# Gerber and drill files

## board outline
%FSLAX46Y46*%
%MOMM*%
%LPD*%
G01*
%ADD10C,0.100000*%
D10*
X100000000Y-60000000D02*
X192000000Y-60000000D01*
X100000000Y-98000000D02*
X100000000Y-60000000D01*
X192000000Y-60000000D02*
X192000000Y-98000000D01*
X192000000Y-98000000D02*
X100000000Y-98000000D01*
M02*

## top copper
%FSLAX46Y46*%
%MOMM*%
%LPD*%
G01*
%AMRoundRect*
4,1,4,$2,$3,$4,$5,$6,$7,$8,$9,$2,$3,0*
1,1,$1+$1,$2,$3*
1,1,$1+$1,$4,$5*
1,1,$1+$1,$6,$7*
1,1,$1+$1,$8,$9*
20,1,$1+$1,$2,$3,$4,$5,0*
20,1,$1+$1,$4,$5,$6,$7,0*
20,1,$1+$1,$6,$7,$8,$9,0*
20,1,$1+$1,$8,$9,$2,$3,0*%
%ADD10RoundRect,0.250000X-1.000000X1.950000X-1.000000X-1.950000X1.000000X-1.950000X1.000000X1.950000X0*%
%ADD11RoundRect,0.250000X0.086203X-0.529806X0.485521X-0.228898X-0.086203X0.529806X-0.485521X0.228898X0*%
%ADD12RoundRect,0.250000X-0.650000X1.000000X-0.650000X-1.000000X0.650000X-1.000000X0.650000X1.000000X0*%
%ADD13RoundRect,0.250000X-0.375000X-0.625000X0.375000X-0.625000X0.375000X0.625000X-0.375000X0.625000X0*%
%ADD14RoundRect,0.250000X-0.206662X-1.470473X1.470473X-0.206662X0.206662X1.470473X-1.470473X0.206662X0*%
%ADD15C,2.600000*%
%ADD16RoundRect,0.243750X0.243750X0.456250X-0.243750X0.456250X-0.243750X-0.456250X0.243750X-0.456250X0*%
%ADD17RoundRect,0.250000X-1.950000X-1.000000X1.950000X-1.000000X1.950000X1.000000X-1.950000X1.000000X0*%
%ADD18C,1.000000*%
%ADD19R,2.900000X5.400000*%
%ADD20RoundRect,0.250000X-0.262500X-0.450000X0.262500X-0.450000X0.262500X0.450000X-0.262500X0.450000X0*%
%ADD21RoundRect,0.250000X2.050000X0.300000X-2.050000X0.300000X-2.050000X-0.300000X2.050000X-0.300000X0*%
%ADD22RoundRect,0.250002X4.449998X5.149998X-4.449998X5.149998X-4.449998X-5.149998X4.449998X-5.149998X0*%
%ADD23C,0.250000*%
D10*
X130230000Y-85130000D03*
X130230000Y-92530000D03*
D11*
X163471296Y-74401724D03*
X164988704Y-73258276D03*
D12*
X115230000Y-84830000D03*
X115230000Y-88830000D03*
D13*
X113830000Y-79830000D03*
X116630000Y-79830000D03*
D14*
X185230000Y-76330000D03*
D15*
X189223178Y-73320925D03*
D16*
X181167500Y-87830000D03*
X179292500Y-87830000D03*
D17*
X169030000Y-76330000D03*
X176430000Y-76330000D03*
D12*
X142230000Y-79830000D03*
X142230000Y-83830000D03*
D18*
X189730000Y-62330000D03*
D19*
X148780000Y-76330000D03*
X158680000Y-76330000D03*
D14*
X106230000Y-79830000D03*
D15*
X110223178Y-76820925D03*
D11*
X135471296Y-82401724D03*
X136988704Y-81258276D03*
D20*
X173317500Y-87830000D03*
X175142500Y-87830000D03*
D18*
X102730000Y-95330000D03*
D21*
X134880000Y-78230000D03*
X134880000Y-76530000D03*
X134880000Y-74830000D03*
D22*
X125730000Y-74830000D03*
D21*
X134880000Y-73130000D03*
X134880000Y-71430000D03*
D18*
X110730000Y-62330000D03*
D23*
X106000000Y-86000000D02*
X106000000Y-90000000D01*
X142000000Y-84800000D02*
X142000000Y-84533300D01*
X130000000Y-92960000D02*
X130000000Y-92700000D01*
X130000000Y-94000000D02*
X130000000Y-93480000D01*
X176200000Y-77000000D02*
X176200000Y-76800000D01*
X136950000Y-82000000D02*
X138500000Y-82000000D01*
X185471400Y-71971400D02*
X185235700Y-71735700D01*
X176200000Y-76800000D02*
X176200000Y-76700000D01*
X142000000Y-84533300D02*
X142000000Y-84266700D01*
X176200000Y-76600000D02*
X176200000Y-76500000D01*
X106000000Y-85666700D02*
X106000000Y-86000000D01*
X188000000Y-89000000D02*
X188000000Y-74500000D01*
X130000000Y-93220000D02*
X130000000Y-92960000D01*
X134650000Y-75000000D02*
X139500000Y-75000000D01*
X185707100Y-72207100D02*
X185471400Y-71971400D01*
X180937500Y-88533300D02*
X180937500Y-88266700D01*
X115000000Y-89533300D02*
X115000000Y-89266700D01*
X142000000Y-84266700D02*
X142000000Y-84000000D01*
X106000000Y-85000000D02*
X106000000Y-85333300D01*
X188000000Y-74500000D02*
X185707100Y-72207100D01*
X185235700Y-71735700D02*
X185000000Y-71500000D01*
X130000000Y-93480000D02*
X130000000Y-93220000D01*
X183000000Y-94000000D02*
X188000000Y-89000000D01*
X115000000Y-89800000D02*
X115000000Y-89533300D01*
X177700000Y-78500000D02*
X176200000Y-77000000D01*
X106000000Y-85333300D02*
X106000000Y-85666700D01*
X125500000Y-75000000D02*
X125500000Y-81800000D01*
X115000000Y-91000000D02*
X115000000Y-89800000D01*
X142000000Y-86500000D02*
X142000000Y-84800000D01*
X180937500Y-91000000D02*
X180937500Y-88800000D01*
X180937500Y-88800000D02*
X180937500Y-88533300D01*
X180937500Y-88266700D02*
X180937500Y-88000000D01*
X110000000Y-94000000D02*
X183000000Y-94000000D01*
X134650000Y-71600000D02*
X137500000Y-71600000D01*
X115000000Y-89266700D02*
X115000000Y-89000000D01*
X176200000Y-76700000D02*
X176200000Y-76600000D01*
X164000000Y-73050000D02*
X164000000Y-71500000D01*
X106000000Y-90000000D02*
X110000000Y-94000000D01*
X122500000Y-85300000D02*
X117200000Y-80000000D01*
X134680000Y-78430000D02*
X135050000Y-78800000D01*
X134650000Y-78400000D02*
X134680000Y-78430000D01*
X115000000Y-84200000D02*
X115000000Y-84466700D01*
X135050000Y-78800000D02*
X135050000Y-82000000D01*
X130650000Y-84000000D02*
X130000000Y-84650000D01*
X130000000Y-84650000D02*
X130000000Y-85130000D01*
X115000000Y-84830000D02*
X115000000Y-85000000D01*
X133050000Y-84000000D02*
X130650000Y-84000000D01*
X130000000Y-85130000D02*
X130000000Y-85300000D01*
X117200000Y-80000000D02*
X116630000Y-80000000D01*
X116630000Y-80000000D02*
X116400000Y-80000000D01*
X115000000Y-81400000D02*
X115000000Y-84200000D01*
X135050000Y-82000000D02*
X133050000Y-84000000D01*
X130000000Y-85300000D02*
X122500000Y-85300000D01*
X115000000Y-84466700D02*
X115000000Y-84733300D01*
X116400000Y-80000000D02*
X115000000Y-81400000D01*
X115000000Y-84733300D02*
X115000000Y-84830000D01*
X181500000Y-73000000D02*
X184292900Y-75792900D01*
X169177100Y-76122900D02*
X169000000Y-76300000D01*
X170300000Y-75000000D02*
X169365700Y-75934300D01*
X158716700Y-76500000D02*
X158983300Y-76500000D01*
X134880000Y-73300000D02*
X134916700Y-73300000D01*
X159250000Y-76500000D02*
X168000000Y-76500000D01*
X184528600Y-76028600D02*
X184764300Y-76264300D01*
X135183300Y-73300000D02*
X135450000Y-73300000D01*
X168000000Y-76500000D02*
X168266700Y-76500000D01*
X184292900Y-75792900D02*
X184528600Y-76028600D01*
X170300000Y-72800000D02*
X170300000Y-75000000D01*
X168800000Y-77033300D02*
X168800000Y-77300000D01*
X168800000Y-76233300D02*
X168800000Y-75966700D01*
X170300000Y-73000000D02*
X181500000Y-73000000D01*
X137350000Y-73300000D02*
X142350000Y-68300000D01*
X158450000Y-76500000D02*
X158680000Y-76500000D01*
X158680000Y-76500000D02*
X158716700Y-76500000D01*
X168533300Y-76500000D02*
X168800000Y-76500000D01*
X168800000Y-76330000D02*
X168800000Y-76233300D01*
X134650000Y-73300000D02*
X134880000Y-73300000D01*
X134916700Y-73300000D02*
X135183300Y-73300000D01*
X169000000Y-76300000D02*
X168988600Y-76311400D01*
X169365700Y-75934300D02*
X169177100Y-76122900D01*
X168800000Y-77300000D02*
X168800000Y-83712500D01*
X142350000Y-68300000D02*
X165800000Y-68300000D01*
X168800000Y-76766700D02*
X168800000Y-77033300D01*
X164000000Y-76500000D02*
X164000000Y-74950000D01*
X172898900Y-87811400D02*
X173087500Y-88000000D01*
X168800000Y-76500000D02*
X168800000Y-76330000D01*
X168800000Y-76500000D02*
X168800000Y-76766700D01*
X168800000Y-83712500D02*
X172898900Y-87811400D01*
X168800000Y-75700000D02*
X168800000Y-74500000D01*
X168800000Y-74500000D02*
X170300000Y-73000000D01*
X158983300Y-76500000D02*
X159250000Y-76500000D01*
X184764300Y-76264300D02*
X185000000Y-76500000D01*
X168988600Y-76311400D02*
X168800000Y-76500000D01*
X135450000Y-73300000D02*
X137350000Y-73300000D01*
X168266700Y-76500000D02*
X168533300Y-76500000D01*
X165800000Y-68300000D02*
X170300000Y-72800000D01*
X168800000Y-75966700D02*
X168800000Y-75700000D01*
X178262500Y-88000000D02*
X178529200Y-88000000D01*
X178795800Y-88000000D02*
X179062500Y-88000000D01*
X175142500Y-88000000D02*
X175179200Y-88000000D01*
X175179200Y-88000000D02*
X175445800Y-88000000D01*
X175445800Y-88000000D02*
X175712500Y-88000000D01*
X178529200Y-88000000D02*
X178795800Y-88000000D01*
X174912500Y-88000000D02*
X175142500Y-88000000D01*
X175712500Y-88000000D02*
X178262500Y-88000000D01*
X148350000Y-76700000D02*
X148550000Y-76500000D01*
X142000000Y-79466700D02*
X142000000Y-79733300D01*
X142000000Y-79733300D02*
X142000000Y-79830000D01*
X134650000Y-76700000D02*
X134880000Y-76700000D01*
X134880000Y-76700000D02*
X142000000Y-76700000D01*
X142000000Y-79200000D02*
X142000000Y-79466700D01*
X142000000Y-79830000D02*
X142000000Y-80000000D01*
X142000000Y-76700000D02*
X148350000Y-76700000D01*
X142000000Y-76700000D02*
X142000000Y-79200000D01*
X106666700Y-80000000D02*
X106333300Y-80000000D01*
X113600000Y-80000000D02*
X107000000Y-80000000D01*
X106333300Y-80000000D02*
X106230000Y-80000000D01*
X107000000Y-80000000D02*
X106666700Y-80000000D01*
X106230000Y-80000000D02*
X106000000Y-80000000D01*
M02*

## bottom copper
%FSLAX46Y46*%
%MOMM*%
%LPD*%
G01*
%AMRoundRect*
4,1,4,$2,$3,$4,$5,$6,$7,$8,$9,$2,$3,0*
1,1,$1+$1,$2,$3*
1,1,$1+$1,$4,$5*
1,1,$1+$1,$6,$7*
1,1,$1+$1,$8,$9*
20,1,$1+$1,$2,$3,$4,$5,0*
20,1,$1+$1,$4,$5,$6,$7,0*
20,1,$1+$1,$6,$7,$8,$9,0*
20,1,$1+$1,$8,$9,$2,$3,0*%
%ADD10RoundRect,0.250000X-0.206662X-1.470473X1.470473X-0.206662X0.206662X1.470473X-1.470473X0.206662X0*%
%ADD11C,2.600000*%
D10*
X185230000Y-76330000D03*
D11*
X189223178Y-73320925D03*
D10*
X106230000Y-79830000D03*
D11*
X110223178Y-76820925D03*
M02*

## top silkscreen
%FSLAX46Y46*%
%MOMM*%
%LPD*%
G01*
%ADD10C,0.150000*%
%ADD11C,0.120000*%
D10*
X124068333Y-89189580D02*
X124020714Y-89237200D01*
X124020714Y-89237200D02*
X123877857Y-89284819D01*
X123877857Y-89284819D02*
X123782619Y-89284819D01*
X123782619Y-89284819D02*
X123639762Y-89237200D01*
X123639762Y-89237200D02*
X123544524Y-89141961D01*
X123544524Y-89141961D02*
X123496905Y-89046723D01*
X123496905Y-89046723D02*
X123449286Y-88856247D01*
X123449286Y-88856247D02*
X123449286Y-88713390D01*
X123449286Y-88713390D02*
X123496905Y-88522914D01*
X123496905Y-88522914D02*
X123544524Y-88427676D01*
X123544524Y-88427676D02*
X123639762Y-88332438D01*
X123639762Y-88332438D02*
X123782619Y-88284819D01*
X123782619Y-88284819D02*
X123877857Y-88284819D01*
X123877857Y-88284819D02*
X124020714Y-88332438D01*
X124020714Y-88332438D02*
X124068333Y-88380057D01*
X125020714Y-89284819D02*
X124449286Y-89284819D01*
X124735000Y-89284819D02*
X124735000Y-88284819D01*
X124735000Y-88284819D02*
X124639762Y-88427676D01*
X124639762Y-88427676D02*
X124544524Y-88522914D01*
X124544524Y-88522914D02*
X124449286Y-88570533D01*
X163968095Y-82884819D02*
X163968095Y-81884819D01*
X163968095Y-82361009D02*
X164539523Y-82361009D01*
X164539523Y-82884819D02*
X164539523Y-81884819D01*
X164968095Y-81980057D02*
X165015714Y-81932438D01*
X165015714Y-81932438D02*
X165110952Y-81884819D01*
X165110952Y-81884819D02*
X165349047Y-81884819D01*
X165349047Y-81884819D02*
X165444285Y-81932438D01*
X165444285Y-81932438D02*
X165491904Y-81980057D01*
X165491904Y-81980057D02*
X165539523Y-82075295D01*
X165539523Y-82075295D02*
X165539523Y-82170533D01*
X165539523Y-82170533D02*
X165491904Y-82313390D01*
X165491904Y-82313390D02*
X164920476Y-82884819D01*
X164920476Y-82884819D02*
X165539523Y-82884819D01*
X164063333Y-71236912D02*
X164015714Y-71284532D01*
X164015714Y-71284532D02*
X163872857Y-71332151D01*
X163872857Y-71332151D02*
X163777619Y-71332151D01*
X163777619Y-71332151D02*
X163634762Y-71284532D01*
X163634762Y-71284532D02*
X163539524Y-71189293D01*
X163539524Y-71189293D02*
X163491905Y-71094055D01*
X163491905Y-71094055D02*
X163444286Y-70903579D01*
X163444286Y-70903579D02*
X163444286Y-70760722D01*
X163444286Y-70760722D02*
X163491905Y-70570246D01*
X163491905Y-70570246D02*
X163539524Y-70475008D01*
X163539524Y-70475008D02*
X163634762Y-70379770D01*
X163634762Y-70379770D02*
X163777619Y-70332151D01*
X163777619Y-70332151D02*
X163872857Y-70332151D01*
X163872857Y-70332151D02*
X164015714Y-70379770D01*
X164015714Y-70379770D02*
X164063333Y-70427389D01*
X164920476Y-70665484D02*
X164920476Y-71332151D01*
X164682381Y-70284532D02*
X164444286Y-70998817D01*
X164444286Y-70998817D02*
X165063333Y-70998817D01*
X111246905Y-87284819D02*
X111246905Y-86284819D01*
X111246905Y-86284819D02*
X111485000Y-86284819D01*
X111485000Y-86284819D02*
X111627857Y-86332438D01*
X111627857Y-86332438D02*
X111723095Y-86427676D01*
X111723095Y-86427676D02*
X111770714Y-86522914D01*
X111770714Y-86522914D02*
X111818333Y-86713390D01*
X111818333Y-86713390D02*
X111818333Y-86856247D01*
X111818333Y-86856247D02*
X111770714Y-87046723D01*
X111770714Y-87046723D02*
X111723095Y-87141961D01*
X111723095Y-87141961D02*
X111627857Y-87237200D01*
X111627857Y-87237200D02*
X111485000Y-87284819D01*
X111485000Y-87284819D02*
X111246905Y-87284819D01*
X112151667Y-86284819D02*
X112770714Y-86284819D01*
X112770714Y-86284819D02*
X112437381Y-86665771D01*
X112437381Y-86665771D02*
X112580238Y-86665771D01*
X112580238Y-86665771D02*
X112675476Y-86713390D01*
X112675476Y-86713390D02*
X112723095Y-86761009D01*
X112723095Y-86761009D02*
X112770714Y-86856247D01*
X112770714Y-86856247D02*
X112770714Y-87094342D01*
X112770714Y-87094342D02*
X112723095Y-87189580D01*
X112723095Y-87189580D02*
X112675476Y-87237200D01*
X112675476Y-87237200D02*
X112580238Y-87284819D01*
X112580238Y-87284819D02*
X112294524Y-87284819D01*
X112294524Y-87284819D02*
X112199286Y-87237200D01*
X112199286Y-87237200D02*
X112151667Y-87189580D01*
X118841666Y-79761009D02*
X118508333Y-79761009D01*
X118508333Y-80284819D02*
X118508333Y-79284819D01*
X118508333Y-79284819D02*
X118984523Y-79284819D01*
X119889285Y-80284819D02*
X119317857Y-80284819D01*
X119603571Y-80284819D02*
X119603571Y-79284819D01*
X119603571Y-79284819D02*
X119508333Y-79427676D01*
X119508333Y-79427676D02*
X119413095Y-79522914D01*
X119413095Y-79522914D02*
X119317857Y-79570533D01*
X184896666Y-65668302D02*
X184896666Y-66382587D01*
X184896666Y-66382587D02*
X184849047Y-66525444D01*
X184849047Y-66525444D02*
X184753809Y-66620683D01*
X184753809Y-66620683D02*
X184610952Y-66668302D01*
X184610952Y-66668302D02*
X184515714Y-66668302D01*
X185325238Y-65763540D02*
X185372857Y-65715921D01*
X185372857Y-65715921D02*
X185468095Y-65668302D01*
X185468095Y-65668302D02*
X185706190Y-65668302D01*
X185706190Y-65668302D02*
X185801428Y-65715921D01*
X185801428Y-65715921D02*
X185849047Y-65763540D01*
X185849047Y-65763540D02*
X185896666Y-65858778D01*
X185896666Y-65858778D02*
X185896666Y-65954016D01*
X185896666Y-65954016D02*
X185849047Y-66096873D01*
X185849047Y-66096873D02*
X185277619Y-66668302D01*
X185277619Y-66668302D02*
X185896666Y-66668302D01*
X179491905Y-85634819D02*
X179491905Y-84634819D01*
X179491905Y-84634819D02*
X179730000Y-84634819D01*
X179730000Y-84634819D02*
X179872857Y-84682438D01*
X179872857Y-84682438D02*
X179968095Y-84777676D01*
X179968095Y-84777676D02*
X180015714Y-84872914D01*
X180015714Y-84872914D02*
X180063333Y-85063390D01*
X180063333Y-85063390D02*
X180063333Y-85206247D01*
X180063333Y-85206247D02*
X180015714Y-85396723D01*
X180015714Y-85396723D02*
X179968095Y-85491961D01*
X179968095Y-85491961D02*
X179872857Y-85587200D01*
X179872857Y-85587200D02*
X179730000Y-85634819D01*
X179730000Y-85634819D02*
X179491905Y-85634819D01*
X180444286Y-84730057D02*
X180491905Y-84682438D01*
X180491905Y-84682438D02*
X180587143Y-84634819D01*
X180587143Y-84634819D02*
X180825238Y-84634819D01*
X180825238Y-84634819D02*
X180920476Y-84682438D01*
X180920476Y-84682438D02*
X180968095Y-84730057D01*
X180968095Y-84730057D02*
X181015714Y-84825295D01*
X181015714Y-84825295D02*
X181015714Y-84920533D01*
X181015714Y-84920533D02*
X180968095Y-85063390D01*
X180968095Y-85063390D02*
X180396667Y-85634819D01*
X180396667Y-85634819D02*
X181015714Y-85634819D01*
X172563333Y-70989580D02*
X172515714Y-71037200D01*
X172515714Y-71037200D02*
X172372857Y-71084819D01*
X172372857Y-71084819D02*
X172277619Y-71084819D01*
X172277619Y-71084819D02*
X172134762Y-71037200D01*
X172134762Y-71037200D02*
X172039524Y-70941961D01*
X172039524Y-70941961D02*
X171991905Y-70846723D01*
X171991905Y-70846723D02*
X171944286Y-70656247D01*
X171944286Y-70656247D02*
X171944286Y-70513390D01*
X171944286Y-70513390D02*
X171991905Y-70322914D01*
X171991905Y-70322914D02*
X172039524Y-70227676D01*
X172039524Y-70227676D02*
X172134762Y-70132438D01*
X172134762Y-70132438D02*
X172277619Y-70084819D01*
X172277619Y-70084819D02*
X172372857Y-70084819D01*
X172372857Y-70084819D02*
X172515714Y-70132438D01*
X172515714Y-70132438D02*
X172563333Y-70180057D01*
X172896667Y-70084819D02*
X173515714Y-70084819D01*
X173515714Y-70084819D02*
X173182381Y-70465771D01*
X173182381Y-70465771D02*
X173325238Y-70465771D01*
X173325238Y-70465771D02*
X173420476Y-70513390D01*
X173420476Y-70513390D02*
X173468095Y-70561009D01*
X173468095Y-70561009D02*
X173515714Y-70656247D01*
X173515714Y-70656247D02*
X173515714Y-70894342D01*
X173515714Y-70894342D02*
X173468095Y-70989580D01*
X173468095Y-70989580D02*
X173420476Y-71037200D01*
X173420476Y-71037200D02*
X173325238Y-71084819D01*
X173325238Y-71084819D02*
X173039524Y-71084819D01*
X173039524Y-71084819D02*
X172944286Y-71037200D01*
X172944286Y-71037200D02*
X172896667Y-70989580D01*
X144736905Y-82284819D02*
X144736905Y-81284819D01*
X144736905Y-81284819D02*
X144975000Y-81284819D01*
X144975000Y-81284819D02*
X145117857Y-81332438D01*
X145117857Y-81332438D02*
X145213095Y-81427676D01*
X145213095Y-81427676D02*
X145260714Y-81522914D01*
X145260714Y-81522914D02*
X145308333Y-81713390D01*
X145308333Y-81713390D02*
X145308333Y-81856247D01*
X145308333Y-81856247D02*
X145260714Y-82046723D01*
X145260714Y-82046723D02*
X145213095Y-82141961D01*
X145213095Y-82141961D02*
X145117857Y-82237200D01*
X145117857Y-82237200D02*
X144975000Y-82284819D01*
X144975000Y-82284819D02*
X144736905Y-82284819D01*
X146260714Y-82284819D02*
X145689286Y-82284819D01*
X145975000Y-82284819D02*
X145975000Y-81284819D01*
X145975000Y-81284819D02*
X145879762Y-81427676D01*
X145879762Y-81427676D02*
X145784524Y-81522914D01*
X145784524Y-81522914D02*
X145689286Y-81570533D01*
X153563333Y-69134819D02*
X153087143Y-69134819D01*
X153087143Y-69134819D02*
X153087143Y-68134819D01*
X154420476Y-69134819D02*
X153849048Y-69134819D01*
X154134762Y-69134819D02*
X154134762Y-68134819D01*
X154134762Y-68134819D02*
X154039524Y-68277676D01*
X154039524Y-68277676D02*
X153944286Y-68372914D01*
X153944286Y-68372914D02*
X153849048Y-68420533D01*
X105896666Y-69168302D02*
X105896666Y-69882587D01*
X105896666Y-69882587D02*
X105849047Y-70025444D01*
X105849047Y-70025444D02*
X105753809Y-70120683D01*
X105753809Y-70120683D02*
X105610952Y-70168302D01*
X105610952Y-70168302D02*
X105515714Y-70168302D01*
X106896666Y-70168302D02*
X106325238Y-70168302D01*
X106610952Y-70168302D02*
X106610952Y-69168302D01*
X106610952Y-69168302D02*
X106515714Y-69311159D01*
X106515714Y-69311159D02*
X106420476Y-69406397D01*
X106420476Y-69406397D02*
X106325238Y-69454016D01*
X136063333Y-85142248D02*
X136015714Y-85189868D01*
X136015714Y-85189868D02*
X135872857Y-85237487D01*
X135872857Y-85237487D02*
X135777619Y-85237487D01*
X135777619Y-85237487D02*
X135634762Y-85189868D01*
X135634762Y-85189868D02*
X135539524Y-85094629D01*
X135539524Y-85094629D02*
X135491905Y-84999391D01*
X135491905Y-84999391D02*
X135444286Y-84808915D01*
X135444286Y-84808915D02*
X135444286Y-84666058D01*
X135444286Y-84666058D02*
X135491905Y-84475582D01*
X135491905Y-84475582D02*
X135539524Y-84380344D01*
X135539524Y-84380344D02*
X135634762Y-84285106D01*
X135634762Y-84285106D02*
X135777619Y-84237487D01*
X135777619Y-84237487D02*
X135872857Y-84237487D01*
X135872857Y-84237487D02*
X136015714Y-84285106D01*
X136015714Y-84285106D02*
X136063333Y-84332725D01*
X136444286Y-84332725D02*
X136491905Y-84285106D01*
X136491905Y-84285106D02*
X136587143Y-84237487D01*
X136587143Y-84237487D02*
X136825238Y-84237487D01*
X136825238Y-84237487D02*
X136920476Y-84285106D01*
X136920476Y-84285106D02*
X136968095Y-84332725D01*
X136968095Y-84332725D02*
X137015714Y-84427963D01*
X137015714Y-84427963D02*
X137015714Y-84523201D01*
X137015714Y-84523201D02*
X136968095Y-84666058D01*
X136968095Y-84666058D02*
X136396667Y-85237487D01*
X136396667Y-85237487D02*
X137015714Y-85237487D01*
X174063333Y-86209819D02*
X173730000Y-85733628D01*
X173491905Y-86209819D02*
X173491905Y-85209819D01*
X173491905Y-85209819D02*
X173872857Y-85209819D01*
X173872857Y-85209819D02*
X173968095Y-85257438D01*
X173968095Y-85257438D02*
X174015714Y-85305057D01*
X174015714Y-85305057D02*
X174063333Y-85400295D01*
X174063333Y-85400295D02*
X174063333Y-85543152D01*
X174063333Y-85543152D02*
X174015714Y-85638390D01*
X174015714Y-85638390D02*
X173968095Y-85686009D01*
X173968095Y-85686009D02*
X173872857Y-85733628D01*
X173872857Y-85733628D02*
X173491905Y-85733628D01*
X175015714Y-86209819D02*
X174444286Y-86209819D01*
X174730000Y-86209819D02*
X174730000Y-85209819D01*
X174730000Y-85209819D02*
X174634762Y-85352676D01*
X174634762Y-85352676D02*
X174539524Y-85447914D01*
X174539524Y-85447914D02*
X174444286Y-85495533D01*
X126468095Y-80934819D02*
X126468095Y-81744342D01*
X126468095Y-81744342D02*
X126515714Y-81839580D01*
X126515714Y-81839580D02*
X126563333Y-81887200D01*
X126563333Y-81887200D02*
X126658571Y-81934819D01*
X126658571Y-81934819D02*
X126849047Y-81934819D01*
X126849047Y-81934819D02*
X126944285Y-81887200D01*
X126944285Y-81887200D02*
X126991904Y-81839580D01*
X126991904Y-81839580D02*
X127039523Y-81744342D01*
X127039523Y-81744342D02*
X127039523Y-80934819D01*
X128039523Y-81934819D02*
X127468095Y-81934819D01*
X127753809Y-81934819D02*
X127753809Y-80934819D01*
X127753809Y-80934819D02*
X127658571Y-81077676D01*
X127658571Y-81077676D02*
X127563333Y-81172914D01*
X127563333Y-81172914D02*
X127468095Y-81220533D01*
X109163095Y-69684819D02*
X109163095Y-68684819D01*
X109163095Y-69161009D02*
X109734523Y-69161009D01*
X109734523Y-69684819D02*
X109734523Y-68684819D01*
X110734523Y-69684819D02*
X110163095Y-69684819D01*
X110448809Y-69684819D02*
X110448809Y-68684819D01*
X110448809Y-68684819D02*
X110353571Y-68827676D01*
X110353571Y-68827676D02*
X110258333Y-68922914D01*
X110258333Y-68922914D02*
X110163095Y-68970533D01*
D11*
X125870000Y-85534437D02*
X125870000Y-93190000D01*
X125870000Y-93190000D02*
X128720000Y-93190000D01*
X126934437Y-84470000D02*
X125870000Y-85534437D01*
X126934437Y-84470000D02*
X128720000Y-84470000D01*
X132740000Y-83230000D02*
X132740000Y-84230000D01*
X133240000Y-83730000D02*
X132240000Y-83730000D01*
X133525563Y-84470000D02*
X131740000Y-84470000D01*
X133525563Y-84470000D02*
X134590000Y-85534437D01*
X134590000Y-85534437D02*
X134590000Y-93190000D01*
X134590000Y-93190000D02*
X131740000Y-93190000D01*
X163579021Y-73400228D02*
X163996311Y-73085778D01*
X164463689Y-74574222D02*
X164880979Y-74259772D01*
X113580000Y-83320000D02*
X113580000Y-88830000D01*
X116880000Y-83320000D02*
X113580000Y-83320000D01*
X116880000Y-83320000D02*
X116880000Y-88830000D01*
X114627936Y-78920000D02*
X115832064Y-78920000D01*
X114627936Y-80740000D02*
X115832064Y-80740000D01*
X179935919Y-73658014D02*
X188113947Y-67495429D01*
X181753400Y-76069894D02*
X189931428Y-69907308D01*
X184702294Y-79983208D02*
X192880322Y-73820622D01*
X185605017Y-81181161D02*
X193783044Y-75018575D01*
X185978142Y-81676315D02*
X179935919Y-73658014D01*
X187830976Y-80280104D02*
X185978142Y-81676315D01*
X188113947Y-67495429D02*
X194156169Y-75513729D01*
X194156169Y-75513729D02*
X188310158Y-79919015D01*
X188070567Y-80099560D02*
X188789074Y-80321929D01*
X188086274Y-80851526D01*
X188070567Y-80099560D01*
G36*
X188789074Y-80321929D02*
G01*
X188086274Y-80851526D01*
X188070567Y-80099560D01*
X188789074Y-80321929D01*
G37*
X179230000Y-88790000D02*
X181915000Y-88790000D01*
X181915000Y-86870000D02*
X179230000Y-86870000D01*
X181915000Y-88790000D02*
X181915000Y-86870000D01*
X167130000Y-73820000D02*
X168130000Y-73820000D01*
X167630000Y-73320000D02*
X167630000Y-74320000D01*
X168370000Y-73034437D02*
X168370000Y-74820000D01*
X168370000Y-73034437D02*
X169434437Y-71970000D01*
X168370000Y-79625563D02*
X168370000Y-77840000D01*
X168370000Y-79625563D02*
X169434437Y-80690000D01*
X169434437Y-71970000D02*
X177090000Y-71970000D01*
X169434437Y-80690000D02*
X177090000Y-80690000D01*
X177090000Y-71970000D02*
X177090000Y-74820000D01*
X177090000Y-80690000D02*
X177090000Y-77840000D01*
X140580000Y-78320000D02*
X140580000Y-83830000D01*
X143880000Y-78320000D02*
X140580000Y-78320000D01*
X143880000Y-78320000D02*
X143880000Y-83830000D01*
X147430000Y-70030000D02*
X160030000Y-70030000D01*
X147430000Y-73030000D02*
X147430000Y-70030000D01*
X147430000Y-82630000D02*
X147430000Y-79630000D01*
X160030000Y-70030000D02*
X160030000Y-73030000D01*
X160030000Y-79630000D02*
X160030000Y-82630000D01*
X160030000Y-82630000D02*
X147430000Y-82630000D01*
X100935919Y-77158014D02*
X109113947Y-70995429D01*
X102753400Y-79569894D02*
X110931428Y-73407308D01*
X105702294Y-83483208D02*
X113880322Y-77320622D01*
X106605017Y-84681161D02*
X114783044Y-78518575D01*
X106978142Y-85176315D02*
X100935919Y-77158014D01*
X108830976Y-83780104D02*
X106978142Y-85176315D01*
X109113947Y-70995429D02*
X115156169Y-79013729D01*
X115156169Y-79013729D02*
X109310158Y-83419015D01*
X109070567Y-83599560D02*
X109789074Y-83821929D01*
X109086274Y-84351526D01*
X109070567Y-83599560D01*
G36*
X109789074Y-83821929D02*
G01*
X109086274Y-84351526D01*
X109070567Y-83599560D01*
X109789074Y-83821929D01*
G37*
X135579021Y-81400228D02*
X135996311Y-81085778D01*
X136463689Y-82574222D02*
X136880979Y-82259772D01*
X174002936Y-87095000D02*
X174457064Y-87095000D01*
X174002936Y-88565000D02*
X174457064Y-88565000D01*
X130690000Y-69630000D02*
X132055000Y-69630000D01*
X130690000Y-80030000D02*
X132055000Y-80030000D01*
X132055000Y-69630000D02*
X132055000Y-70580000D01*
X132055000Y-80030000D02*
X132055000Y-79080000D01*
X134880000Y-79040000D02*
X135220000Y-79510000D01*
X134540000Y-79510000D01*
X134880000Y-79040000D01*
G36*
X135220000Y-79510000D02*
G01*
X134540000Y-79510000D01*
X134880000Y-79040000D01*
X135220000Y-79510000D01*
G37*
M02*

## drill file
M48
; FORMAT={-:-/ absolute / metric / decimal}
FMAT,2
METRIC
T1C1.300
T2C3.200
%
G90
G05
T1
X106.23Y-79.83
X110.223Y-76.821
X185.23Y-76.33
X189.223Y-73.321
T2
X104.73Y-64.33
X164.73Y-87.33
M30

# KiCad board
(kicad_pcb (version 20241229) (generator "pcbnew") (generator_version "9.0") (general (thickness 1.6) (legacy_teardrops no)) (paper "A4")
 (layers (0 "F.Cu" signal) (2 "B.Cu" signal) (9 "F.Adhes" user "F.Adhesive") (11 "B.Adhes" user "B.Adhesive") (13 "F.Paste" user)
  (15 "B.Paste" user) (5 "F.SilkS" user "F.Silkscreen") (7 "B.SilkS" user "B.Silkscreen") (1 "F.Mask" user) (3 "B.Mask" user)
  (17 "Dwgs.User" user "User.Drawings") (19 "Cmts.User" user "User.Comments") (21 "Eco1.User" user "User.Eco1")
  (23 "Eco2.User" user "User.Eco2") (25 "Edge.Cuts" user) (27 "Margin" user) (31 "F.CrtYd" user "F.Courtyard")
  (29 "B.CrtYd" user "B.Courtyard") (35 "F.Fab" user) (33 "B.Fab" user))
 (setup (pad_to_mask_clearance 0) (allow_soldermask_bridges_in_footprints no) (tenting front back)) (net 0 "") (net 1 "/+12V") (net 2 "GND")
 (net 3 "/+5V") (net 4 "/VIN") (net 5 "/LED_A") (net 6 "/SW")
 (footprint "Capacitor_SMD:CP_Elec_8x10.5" (layer "F.Cu") (at 130.23 88.83 -90)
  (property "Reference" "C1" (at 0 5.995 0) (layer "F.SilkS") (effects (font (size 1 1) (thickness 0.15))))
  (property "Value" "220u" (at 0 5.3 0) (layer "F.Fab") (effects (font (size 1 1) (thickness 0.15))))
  (fp_line (start -3.295563 4.36) (end 4.36 4.36) (stroke (width 0.12) (type solid)) (layer "F.SilkS"))
  (fp_line (start 4.36 4.36) (end 4.36 1.51) (stroke (width 0.12) (type solid)) (layer "F.SilkS"))
  (fp_line (start -4.36 3.295563) (end -3.295563 4.36) (stroke (width 0.12) (type solid)) (layer "F.SilkS"))
  (fp_line (start -4.36 3.295563) (end -4.36 1.51) (stroke (width 0.12) (type solid)) (layer "F.SilkS"))
  (fp_line (start -5.6 -2.51) (end -4.6 -2.51) (stroke (width 0.12) (type solid)) (layer "F.SilkS"))
  (fp_line (start -5.1 -3.01) (end -5.1 -2.01) (stroke (width 0.12) (type solid)) (layer "F.SilkS"))
  (fp_line (start -4.36 -3.295563) (end -4.36 -1.51) (stroke (width 0.12) (type solid)) (layer "F.SilkS"))
  (fp_line (start -4.36 -3.295563) (end -3.295563 -4.36) (stroke (width 0.12) (type solid)) (layer "F.SilkS"))
  (fp_line (start -3.295563 -4.36) (end 4.36 -4.36) (stroke (width 0.12) (type solid)) (layer "F.SilkS"))
  (fp_line (start 4.36 -4.36) (end 4.36 -1.51) (stroke (width 0.12) (type solid)) (layer "F.SilkS"))
  (pad "1" smd roundrect (at -3.7 0 270) (size 4.4 2.5) (layers "F.Cu" "F.Mask" "F.Paste") (roundrect_rratio 0.1) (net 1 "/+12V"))
  (pad "2" smd roundrect (at 3.7 0 270) (size 4.4 2.5) (layers "F.Cu" "F.Mask" "F.Paste") (roundrect_rratio 0.1) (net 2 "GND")
   (zone_connect 1) (thermal_bridge_width 1)))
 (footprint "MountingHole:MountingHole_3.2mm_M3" (layer "F.Cu") (at 164.73 87.33)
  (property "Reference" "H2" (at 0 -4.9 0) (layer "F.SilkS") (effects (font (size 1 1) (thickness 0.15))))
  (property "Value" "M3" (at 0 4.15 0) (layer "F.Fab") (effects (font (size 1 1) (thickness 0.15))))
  (pad "" np_thru_hole circle (at 0 0) (size 3.2 3.2) (drill 3.2) (layers "*.Cu" "*.Mask")))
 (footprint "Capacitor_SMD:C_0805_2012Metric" (layer "F.Cu") (at 164.23 73.83 37)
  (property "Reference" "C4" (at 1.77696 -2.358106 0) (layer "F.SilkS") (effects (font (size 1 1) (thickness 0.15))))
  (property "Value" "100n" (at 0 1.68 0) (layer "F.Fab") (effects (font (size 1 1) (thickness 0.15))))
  (fp_line (start -0.261252 -0.735) (end 0.261252 -0.735) (stroke (width 0.12) (type solid)) (layer "F.SilkS"))
  (fp_line (start -0.261252 0.735) (end 0.261252 0.735) (stroke (width 0.12) (type solid)) (layer "F.SilkS"))
  (pad "1" smd roundrect (at -0.95 0 37) (size 1 1.45) (layers "F.Cu" "F.Mask" "F.Paste") (roundrect_rratio 0.25) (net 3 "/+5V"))
  (pad "2" smd roundrect (at 0.95 0 37) (size 1 1.45) (layers "F.Cu" "F.Mask" "F.Paste") (roundrect_rratio 0.25) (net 2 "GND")))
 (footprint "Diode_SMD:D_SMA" (layer "F.Cu") (at 115.23 86.83 -90)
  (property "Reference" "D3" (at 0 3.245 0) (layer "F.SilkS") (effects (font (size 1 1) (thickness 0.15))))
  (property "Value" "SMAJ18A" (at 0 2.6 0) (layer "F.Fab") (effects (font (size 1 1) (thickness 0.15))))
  (fp_line (start -3.51 1.65) (end 2 1.65) (stroke (width 0.12) (type solid)) (layer "F.SilkS"))
  (fp_line (start -3.51 -1.65) (end -3.51 1.65) (stroke (width 0.12) (type solid)) (layer "F.SilkS"))
  (fp_line (start -3.51 -1.65) (end 2 -1.65) (stroke (width 0.12) (type solid)) (layer "F.SilkS"))
  (pad "1" smd roundrect (at -2 0 270) (size 2.5 1.8) (layers "F.Cu" "F.Mask" "F.Paste") (roundrect_rratio 0.1388888889) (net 1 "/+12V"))
  (pad "2" smd roundrect (at 2 0 270) (size 2.5 1.8) (layers "F.Cu" "F.Mask" "F.Paste") (roundrect_rratio 0.1388888889) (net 2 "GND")))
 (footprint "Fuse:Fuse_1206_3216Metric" (layer "F.Cu") (at 115.23 79.83)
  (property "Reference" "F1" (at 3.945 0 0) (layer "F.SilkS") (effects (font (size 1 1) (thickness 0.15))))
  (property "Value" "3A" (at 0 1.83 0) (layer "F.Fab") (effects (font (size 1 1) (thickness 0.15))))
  (fp_line (start -0.602064 -0.91) (end 0.602064 -0.91) (stroke (width 0.12) (type solid)) (layer "F.SilkS"))
  (fp_line (start -0.602064 0.91) (end 0.602064 0.91) (stroke (width 0.12) (type solid)) (layer "F.SilkS"))
  (pad "1" smd roundrect (at -1.4 0) (size 1.25 1.75) (layers "F.Cu" "F.Mask" "F.Paste") (roundrect_rratio 0.2) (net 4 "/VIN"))
  (pad "2" smd roundrect (at 1.4 0) (size 1.25 1.75) (layers "F.Cu" "F.Mask" "F.Paste") (roundrect_rratio 0.2) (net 1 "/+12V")))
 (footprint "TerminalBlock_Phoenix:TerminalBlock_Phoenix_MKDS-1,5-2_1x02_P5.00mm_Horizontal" (layer "F.Cu") (at 185.23 76.33 37)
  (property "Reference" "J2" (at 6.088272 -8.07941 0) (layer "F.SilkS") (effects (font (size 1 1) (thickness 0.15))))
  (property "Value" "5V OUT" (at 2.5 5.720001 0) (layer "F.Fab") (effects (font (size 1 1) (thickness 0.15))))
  (fp_line (start -2.62 -5.32) (end 7.62 -5.319999) (stroke (width 0.12) (type solid)) (layer "F.SilkS"))
  (fp_line (start -2.620001 -2.3) (end 7.62 -2.3) (stroke (width 0.12) (type solid)) (layer "F.SilkS"))
  (fp_line (start -2.62 2.6) (end 7.62 2.6) (stroke (width 0.12) (type solid)) (layer "F.SilkS"))
  (fp_line (start -2.62 4.1) (end 7.62 4.1) (stroke (width 0.12) (type solid)) (layer "F.SilkS"))
  (fp_line (start -2.62 4.72) (end -2.62 -5.32) (stroke (width 0.12) (type solid)) (layer "F.SilkS"))
  (fp_line (start -0.3 4.72) (end -2.62 4.72) (stroke (width 0.12) (type solid)) (layer "F.SilkS"))
  (fp_line (start 7.62 -5.319999) (end 7.62 4.72) (stroke (width 0.12) (type solid)) (layer "F.SilkS"))
  (fp_line (start 7.62 4.72) (end 0.3 4.72) (stroke (width 0.12) (type solid)) (layer "F.SilkS"))
  (fp_poly (pts (xy 0 4.72) (xy 0.44 5.33) (xy -0.44 5.33)) (stroke (width 0.12) (type solid)) (fill yes) (layer "F.SilkS"))
  (pad "1" thru_hole roundrect (at 0 0 37) (size 2.6 2.6) (drill 1.3) (layers "*.Cu" "*.Mask") (remove_unused_layers no)
   (roundrect_rratio 0.096154) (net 3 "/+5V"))
  (pad "2" thru_hole circle (at 5 0 37) (size 2.6 2.6) (drill 1.3) (layers "*.Cu" "*.Mask") (remove_unused_layers no) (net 2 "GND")))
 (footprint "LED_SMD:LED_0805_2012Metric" (layer "F.Cu") (at 180.23 87.83 180)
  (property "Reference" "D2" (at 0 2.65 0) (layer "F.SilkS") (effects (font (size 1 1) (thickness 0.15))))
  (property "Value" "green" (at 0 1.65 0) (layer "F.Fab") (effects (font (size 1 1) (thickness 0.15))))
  (fp_line (start 1 -0.96) (end -1.685 -0.96) (stroke (width 0.12) (type solid)) (layer "F.SilkS"))
  (fp_line (start -1.685 0.96) (end 1 0.96) (stroke (width 0.12) (type solid)) (layer "F.SilkS"))
  (fp_line (start -1.685 -0.96) (end -1.685 0.96) (stroke (width 0.12) (type solid)) (layer "F.SilkS"))
  (pad "1" smd roundrect (at -0.9375 0 180) (size 0.975 1.4) (layers "F.Cu" "F.Mask" "F.Paste") (roundrect_rratio 0.25) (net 2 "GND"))
  (pad "2" smd roundrect (at 0.9375 0 180) (size 0.975 1.4) (layers "F.Cu" "F.Mask" "F.Paste") (roundrect_rratio 0.25) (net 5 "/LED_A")))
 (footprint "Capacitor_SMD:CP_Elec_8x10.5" (layer "F.Cu") (at 172.73 76.33)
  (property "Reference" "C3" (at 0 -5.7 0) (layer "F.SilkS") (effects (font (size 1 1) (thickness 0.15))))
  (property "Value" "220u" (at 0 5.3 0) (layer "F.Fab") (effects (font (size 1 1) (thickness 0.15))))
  (fp_line (start -5.6 -2.51) (end -4.6 -2.51) (stroke (width 0.12) (type solid)) (layer "F.SilkS"))
  (fp_line (start -5.1 -3.01) (end -5.1 -2.01) (stroke (width 0.12) (type solid)) (layer "F.SilkS"))
  (fp_line (start -4.36 -3.295563) (end -4.36 -1.51) (stroke (width 0.12) (type solid)) (layer "F.SilkS"))
  (fp_line (start -4.36 -3.295563) (end -3.295563 -4.36) (stroke (width 0.12) (type solid)) (layer "F.SilkS"))
  (fp_line (start -4.36 3.295563) (end -4.36 1.51) (stroke (width 0.12) (type solid)) (layer "F.SilkS"))
  (fp_line (start -4.36 3.295563) (end -3.295563 4.36) (stroke (width 0.12) (type solid)) (layer "F.SilkS"))
  (fp_line (start -3.295563 -4.36) (end 4.36 -4.36) (stroke (width 0.12) (type solid)) (layer "F.SilkS"))
  (fp_line (start -3.295563 4.36) (end 4.36 4.36) (stroke (width 0.12) (type solid)) (layer "F.SilkS"))
  (fp_line (start 4.36 -4.36) (end 4.36 -1.51) (stroke (width 0.12) (type solid)) (layer "F.SilkS"))
  (fp_line (start 4.36 4.36) (end 4.36 1.51) (stroke (width 0.12) (type solid)) (layer "F.SilkS"))
  (pad "1" smd roundrect (at -3.7 0) (size 4.4 2.5) (layers "F.Cu" "F.Mask" "F.Paste") (roundrect_rratio 0.1) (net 3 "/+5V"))
  (pad "2" smd roundrect (at 3.7 0) (size 4.4 2.5) (layers "F.Cu" "F.Mask" "F.Paste") (roundrect_rratio 0.1) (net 2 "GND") (zone_connect 1)
   (thermal_bridge_width 1)))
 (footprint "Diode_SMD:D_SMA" (layer "F.Cu") (at 142.23 81.83 -90)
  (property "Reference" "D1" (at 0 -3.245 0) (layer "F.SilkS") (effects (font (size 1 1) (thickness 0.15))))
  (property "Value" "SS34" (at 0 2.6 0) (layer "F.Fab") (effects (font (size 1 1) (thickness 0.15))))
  (fp_line (start -3.51 1.65) (end 2 1.65) (stroke (width 0.12) (type solid)) (layer "F.SilkS"))
  (fp_line (start -3.51 -1.65) (end -3.51 1.65) (stroke (width 0.12) (type solid)) (layer "F.SilkS"))
  (fp_line (start -3.51 -1.65) (end 2 -1.65) (stroke (width 0.12) (type solid)) (layer "F.SilkS"))
  (pad "1" smd roundrect (at -2 0 270) (size 2.5 1.8) (layers "F.Cu" "F.Mask" "F.Paste") (roundrect_rratio 0.1388888889) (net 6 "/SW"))
  (pad "2" smd roundrect (at 2 0 270) (size 2.5 1.8) (layers "F.Cu" "F.Mask" "F.Paste") (roundrect_rratio 0.1388888889) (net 2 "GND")))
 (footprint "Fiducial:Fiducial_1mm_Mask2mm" (layer "F.Cu") (at 189.73 62.33 37)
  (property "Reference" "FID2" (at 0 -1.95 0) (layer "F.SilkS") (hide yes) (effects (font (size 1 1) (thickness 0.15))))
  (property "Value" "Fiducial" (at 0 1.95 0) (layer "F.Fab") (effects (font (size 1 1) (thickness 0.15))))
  (pad "" smd circle (at 0 0 37) (size 1 1) (layers "F.Cu" "F.Mask") (solder_mask_margin 0.5) (clearance 0.6)))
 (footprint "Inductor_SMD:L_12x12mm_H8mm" (layer "F.Cu") (at 153.73 76.33)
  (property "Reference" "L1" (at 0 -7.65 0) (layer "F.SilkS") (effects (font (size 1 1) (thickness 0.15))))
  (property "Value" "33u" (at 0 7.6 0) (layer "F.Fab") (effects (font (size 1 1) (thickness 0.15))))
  (fp_line (start -6.3 -6.3) (end 6.3 -6.3) (stroke (width 0.12) (type solid)) (layer "F.SilkS"))
  (fp_line (start -6.3 -3.3) (end -6.3 -6.3) (stroke (width 0.12) (type solid)) (layer "F.SilkS"))
  (fp_line (start -6.3 6.3) (end -6.3 3.3) (stroke (width 0.12) (type solid)) (layer "F.SilkS"))
  (fp_line (start 6.3 -6.3) (end 6.3 -3.3) (stroke (width 0.12) (type solid)) (layer "F.SilkS"))
  (fp_line (start 6.3 3.3) (end 6.3 6.3) (stroke (width 0.12) (type solid)) (layer "F.SilkS"))
  (fp_line (start 6.3 6.3) (end -6.3 6.3) (stroke (width 0.12) (type solid)) (layer "F.SilkS"))
  (pad "1" smd rect (at -4.95 0) (size 2.9 5.4) (layers "F.Cu" "F.Mask" "F.Paste") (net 6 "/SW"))
  (pad "2" smd rect (at 4.95 0) (size 2.9 5.4) (layers "F.Cu" "F.Mask" "F.Paste") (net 3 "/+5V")))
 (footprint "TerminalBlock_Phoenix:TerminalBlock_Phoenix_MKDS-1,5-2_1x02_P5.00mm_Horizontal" (layer "F.Cu") (at 106.23 79.83 37)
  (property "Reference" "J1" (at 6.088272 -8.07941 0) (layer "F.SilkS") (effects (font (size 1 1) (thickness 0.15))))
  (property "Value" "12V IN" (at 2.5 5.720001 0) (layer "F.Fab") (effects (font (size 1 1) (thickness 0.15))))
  (fp_line (start -2.62 -5.32) (end 7.62 -5.319999) (stroke (width 0.12) (type solid)) (layer "F.SilkS"))
  (fp_line (start -2.620001 -2.3) (end 7.62 -2.3) (stroke (width 0.12) (type solid)) (layer "F.SilkS"))
  (fp_line (start -2.62 2.6) (end 7.62 2.6) (stroke (width 0.12) (type solid)) (layer "F.SilkS"))
  (fp_line (start -2.62 4.1) (end 7.62 4.1) (stroke (width 0.12) (type solid)) (layer "F.SilkS"))
  (fp_line (start -2.62 4.72) (end -2.62 -5.32) (stroke (width 0.12) (type solid)) (layer "F.SilkS"))
  (fp_line (start -0.3 4.72) (end -2.62 4.72) (stroke (width 0.12) (type solid)) (layer "F.SilkS"))
  (fp_line (start 7.62 -5.319999) (end 7.62 4.72) (stroke (width 0.12) (type solid)) (layer "F.SilkS"))
  (fp_line (start 7.62 4.72) (end 0.3 4.72) (stroke (width 0.12) (type solid)) (layer "F.SilkS"))
  (fp_poly (pts (xy 0 4.72) (xy 0.44 5.33) (xy -0.44 5.33)) (stroke (width 0.12) (type solid)) (fill yes) (layer "F.SilkS"))
  (pad "1" thru_hole roundrect (at 0 0 37) (size 2.6 2.6) (drill 1.3) (layers "*.Cu" "*.Mask") (remove_unused_layers no)
   (roundrect_rratio 0.096154) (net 4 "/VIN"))
  (pad "2" thru_hole circle (at 5 0 37) (size 2.6 2.6) (drill 1.3) (layers "*.Cu" "*.Mask") (remove_unused_layers no) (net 2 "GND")))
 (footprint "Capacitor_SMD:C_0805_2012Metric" (layer "F.Cu") (at 136.23 81.83 37)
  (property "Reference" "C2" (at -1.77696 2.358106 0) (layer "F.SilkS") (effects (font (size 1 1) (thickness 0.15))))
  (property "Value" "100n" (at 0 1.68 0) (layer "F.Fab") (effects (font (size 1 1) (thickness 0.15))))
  (fp_line (start -0.261252 -0.735) (end 0.261252 -0.735) (stroke (width 0.12) (type solid)) (layer "F.SilkS"))
  (fp_line (start -0.261252 0.735) (end 0.261252 0.735) (stroke (width 0.12) (type solid)) (layer "F.SilkS"))
  (pad "1" smd roundrect (at -0.95 0 37) (size 1 1.45) (layers "F.Cu" "F.Mask" "F.Paste") (roundrect_rratio 0.25) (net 1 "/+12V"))
  (pad "2" smd roundrect (at 0.95 0 37) (size 1 1.45) (layers "F.Cu" "F.Mask" "F.Paste") (roundrect_rratio 0.25) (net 2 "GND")))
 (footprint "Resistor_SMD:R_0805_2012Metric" (layer "F.Cu") (at 174.23 87.83)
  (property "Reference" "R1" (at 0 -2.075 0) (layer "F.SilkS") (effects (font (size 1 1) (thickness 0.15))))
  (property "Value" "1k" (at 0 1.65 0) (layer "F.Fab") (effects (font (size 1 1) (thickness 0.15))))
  (fp_line (start -0.227064 -0.735) (end 0.227064 -0.735) (stroke (width 0.12) (type solid)) (layer "F.SilkS"))
  (fp_line (start -0.227064 0.735) (end 0.227064 0.735) (stroke (width 0.12) (type solid)) (layer "F.SilkS"))
  (pad "1" smd roundrect (at -0.9125 0) (size 1.025 1.4) (layers "F.Cu" "F.Mask" "F.Paste") (roundrect_rratio 0.243902) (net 3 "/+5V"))
  (pad "2" smd roundrect (at 0.9125 0) (size 1.025 1.4) (layers "F.Cu" "F.Mask" "F.Paste") (roundrect_rratio 0.243902) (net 5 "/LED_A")))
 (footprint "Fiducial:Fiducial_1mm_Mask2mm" (layer "F.Cu") (at 102.73 95.33)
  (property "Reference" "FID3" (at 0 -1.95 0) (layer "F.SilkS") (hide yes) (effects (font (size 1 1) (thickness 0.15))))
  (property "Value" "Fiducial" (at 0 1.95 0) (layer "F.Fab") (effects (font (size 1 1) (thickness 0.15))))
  (pad "" smd circle (at 0 0) (size 1 1) (layers "F.Cu" "F.Mask") (solder_mask_margin 0.5) (clearance 0.6)))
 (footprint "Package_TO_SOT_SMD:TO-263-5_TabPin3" (layer "F.Cu") (at 127.23 74.83 180)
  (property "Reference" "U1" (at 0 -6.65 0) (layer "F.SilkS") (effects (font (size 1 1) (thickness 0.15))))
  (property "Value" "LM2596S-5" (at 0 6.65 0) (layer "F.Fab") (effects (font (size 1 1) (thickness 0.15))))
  (fp_line (start -3.46 5.2) (end -4.825 5.2) (stroke (width 0.12) (type solid)) (layer "F.SilkS"))
  (fp_line (start -3.46 -5.2) (end -4.825 -5.2) (stroke (width 0.12) (type solid)) (layer "F.SilkS"))
  (fp_line (start -4.825 5.2) (end -4.825 4.25) (stroke (width 0.12) (type solid)) (layer "F.SilkS"))
  (fp_line (start -4.825 -5.2) (end -4.825 -4.25) (stroke (width 0.12) (type solid)) (layer "F.SilkS"))
  (fp_poly (pts (xy -7.65 -4.21) (xy -7.99 -4.68) (xy -7.31 -4.68)) (stroke (width 0.12) (type solid)) (fill yes) (layer "F.SilkS"))
  (pad "" smd roundrect (at -0.925 -2.775 180) (size 4.55 5.25) (layers "F.Paste") (roundrect_rratio 0.054945))
  (pad "" smd roundrect (at -0.925 2.775 180) (size 4.55 5.25) (layers "F.Paste") (roundrect_rratio 0.054945))
  (pad "" smd roundrect (at 3.925 -2.775 180) (size 4.55 5.25) (layers "F.Paste") (roundrect_rratio 0.054945))
  (pad "" smd roundrect (at 3.925 2.775 180) (size 4.55 5.25) (layers "F.Paste") (roundrect_rratio 0.054945))
  (pad "1" smd roundrect (at -7.65 -3.4 180) (size 4.6 1.1) (layers "F.Cu" "F.Mask" "F.Paste") (roundrect_rratio 0.227273) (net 1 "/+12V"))
  (pad "2" smd roundrect (at -7.65 -1.7 180) (size 4.6 1.1) (layers "F.Cu" "F.Mask" "F.Paste") (roundrect_rratio 0.227273) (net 6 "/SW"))
  (pad "3" smd roundrect (at -7.65 0 180) (size 4.6 1.1) (layers "F.Cu" "F.Mask" "F.Paste") (roundrect_rratio 0.227273) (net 2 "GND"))
  (pad "3" smd roundrect (at 1.5 0 180) (size 9.4 10.8) (layers "F.Cu" "F.Mask") (roundrect_rratio 0.026596) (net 2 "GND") (zone_connect 1)
   (thermal_bridge_width 1))
  (pad "4" smd roundrect (at -7.65 1.7 180) (size 4.6 1.1) (layers "F.Cu" "F.Mask" "F.Paste") (roundrect_rratio 0.227273) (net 3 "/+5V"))
  (pad "5" smd roundrect (at -7.65 3.4 180) (size 4.6 1.1) (layers "F.Cu" "F.Mask" "F.Paste") (roundrect_rratio 0.227273) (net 2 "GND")))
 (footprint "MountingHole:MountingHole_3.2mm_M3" (layer "F.Cu") (at 104.73 64.33)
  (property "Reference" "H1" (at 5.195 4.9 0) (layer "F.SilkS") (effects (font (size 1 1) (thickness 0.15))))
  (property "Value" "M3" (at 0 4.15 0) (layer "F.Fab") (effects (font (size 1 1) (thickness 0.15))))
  (pad "" np_thru_hole circle (at 0 0) (size 3.2 3.2) (drill 3.2) (layers "*.Cu" "*.Mask")))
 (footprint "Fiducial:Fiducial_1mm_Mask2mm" (layer "F.Cu") (at 110.73 62.33)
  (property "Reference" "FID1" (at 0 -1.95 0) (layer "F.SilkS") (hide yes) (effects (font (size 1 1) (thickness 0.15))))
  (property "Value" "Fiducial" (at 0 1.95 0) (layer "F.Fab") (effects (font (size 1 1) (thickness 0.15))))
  (pad "" smd circle (at 0 0) (size 1 1) (layers "F.Cu" "F.Mask") (solder_mask_margin 0.5) (clearance 0.6)))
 (gr_line (start 100 60) (end 192 60) (stroke (width 0.1) (type default)) (layer "Edge.Cuts"))
 (gr_line (start 100 98) (end 100 60) (stroke (width 0.1) (type default)) (layer "Edge.Cuts"))
 (gr_line (start 192 60) (end 192 98) (stroke (width 0.1) (type default)) (layer "Edge.Cuts"))
 (gr_line (start 192 98) (end 100 98) (stroke (width 0.1) (type default)) (layer "Edge.Cuts"))
 (segment (start 106 86) (end 106 90) (width 0.25) (layer "F.Cu") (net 2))
 (segment (start 142 84.8) (end 142 84.5333) (width 0.25) (layer "F.Cu") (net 2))
 (segment (start 130 92.96) (end 130 92.7) (width 0.25) (layer "F.Cu") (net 2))
 (segment (start 130 94) (end 130 93.48) (width 0.25) (layer "F.Cu") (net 2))
 (segment (start 176.2 77) (end 176.2 76.8) (width 0.25) (layer "F.Cu") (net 2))
 (segment (start 136.95 82) (end 138.5 82) (width 0.25) (layer "F.Cu") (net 2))
 (segment (start 185.4714 71.9714) (end 185.2357 71.7357) (width 0.25) (layer "F.Cu") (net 2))
 (segment (start 176.2 76.8) (end 176.2 76.7) (width 0.25) (layer "F.Cu") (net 2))
 (segment (start 142 84.5333) (end 142 84.2667) (width 0.25) (layer "F.Cu") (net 2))
 (segment (start 176.2 76.6) (end 176.2 76.5) (width 0.25) (layer "F.Cu") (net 2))
 (segment (start 106 85.6667) (end 106 86) (width 0.25) (layer "F.Cu") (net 2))
 (segment (start 188 89) (end 188 74.5) (width 0.25) (layer "F.Cu") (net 2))
 (segment (start 130 93.22) (end 130 92.96) (width 0.25) (layer "F.Cu") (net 2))
 (segment (start 134.65 75) (end 139.5 75) (width 0.25) (layer "F.Cu") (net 2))
 (segment (start 185.7071 72.2071) (end 185.4714 71.9714) (width 0.25) (layer "F.Cu") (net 2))
 (segment (start 180.9375 88.5333) (end 180.9375 88.2667) (width 0.25) (layer "F.Cu") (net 2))
 (segment (start 115 89.5333) (end 115 89.2667) (width 0.25) (layer "F.Cu") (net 2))
 (segment (start 142 84.2667) (end 142 84) (width 0.25) (layer "F.Cu") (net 2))
 (segment (start 106 85) (end 106 85.3333) (width 0.25) (layer "F.Cu") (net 2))
 (segment (start 188 74.5) (end 185.7071 72.2071) (width 0.25) (layer "F.Cu") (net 2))
 (segment (start 185.2357 71.7357) (end 185 71.5) (width 0.25) (layer "F.Cu") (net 2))
 (segment (start 130 93.48) (end 130 93.22) (width 0.25) (layer "F.Cu") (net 2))
 (segment (start 183 94) (end 188 89) (width 0.25) (layer "F.Cu") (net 2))
 (segment (start 115 89.8) (end 115 89.5333) (width 0.25) (layer "F.Cu") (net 2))
 (segment (start 177.7 78.5) (end 176.2 77) (width 0.25) (layer "F.Cu") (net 2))
 (segment (start 106 85.3333) (end 106 85.6667) (width 0.25) (layer "F.Cu") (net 2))
 (segment (start 125.5 75) (end 125.5 81.8) (width 0.25) (layer "F.Cu") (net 2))
 (segment (start 115 91) (end 115 89.8) (width 0.25) (layer "F.Cu") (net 2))
 (segment (start 142 86.5) (end 142 84.8) (width 0.25) (layer "F.Cu") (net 2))
 (segment (start 180.9375 91) (end 180.9375 88.8) (width 0.25) (layer "F.Cu") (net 2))
 (segment (start 180.9375 88.8) (end 180.9375 88.5333) (width 0.25) (layer "F.Cu") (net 2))
 (segment (start 180.9375 88.2667) (end 180.9375 88) (width 0.25) (layer "F.Cu") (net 2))
 (segment (start 110 94) (end 183 94) (width 0.25) (layer "F.Cu") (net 2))
 (segment (start 134.65 71.6) (end 137.5 71.6) (width 0.25) (layer "F.Cu") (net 2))
 (segment (start 115 89.2667) (end 115 89) (width 0.25) (layer "F.Cu") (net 2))
 (segment (start 176.2 76.7) (end 176.2 76.6) (width 0.25) (layer "F.Cu") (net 2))
 (segment (start 164 73.05) (end 164 71.5) (width 0.25) (layer "F.Cu") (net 2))
 (segment (start 106 90) (end 110 94) (width 0.25) (layer "F.Cu") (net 2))
 (segment (start 122.5 85.3) (end 117.2 80) (width 0.25) (layer "F.Cu") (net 1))
 (segment (start 134.68 78.43) (end 135.05 78.8) (width 0.25) (layer "F.Cu") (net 1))
 (segment (start 134.65 78.4) (end 134.68 78.43) (width 0.25) (layer "F.Cu") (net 1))
 (segment (start 115 84.2) (end 115 84.4667) (width 0.25) (layer "F.Cu") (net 1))
 (segment (start 135.05 78.8) (end 135.05 82) (width 0.25) (layer "F.Cu") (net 1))
 (segment (start 130.65 84) (end 130 84.65) (width 0.25) (layer "F.Cu") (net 1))
 (segment (start 130 84.65) (end 130 85.13) (width 0.25) (layer "F.Cu") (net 1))
 (segment (start 115 84.83) (end 115 85) (width 0.25) (layer "F.Cu") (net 1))
 (segment (start 133.05 84) (end 130.65 84) (width 0.25) (layer "F.Cu") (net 1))
 (segment (start 130 85.13) (end 130 85.3) (width 0.25) (layer "F.Cu") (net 1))
 (segment (start 117.2 80) (end 116.63 80) (width 0.25) (layer "F.Cu") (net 1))
 (segment (start 116.63 80) (end 116.4 80) (width 0.25) (layer "F.Cu") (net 1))
 (segment (start 115 81.4) (end 115 84.2) (width 0.25) (layer "F.Cu") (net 1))
 (segment (start 135.05 82) (end 133.05 84) (width 0.25) (layer "F.Cu") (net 1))
 (segment (start 130 85.3) (end 122.5 85.3) (width 0.25) (layer "F.Cu") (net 1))
 (segment (start 115 84.4667) (end 115 84.7333) (width 0.25) (layer "F.Cu") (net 1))
 (segment (start 116.4 80) (end 115 81.4) (width 0.25) (layer "F.Cu") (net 1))
 (segment (start 115 84.7333) (end 115 84.83) (width 0.25) (layer "F.Cu") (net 1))
 (segment (start 181.5 73) (end 184.2929 75.7929) (width 0.25) (layer "F.Cu") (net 3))
 (segment (start 169.1771 76.1229) (end 169 76.3) (width 0.25) (layer "F.Cu") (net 3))
 (segment (start 170.3 75) (end 169.3657 75.9343) (width 0.25) (layer "F.Cu") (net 3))
 (segment (start 158.7167 76.5) (end 158.9833 76.5) (width 0.25) (layer "F.Cu") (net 3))
 (segment (start 134.88 73.3) (end 134.9167 73.3) (width 0.25) (layer "F.Cu") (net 3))
 (segment (start 159.25 76.5) (end 168 76.5) (width 0.25) (layer "F.Cu") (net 3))
 (segment (start 184.5286 76.0286) (end 184.7643 76.2643) (width 0.25) (layer "F.Cu") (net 3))
 (segment (start 135.1833 73.3) (end 135.45 73.3) (width 0.25) (layer "F.Cu") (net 3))
 (segment (start 168 76.5) (end 168.2667 76.5) (width 0.25) (layer "F.Cu") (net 3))
 (segment (start 184.2929 75.7929) (end 184.5286 76.0286) (width 0.25) (layer "F.Cu") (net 3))
 (segment (start 170.3 72.8) (end 170.3 75) (width 0.25) (layer "F.Cu") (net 3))
 (segment (start 168.8 77.0333) (end 168.8 77.3) (width 0.25) (layer "F.Cu") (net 3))
 (segment (start 168.8 76.2333) (end 168.8 75.9667) (width 0.25) (layer "F.Cu") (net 3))
 (segment (start 170.3 73) (end 181.5 73) (width 0.25) (layer "F.Cu") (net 3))
 (segment (start 137.35 73.3) (end 142.35 68.3) (width 0.25) (layer "F.Cu") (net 3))
 (segment (start 158.45 76.5) (end 158.68 76.5) (width 0.25) (layer "F.Cu") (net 3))
 (segment (start 158.68 76.5) (end 158.7167 76.5) (width 0.25) (layer "F.Cu") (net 3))
 (segment (start 168.5333 76.5) (end 168.8 76.5) (width 0.25) (layer "F.Cu") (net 3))
 (segment (start 168.8 76.33) (end 168.8 76.2333) (width 0.25) (layer "F.Cu") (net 3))
 (segment (start 134.65 73.3) (end 134.88 73.3) (width 0.25) (layer "F.Cu") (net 3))
 (segment (start 134.9167 73.3) (end 135.1833 73.3) (width 0.25) (layer "F.Cu") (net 3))
 (segment (start 169 76.3) (end 168.9886 76.3114) (width 0.25) (layer "F.Cu") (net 3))
 (segment (start 169.3657 75.9343) (end 169.1771 76.1229) (width 0.25) (layer "F.Cu") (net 3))
 (segment (start 168.8 77.3) (end 168.8 83.7125) (width 0.25) (layer "F.Cu") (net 3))
 (segment (start 142.35 68.3) (end 165.8 68.3) (width 0.25) (layer "F.Cu") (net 3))
 (segment (start 168.8 76.7667) (end 168.8 77.0333) (width 0.25) (layer "F.Cu") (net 3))
 (segment (start 164 76.5) (end 164 74.95) (width 0.25) (layer "F.Cu") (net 3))
 (segment (start 172.8989 87.8114) (end 173.0875 88) (width 0.25) (layer "F.Cu") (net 3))
 (segment (start 168.8 76.5) (end 168.8 76.33) (width 0.25) (layer "F.Cu") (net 3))
 (segment (start 168.8 76.5) (end 168.8 76.7667) (width 0.25) (layer "F.Cu") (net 3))
 (segment (start 168.8 83.7125) (end 172.8989 87.8114) (width 0.25) (layer "F.Cu") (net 3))
 (segment (start 168.8 75.7) (end 168.8 74.5) (width 0.25) (layer "F.Cu") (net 3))
 (segment (start 168.8 74.5) (end 170.3 73) (width 0.25) (layer "F.Cu") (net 3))
 (segment (start 158.9833 76.5) (end 159.25 76.5) (width 0.25) (layer "F.Cu") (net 3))
 (segment (start 184.7643 76.2643) (end 185 76.5) (width 0.25) (layer "F.Cu") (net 3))
 (segment (start 168.9886 76.3114) (end 168.8 76.5) (width 0.25) (layer "F.Cu") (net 3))
 (segment (start 135.45 73.3) (end 137.35 73.3) (width 0.25) (layer "F.Cu") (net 3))
 (segment (start 168.2667 76.5) (end 168.5333 76.5) (width 0.25) (layer "F.Cu") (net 3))
 (segment (start 165.8 68.3) (end 170.3 72.8) (width 0.25) (layer "F.Cu") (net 3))
 (segment (start 168.8 75.9667) (end 168.8 75.7) (width 0.25) (layer "F.Cu") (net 3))
 (segment (start 178.2625 88) (end 178.5292 88) (width 0.25) (layer "F.Cu") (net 5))
 (segment (start 178.7958 88) (end 179.0625 88) (width 0.25) (layer "F.Cu") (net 5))
 (segment (start 175.1425 88) (end 175.1792 88) (width 0.25) (layer "F.Cu") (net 5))
 (segment (start 175.1792 88) (end 175.4458 88) (width 0.25) (layer "F.Cu") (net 5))
 (segment (start 175.4458 88) (end 175.7125 88) (width 0.25) (layer "F.Cu") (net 5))
 (segment (start 178.5292 88) (end 178.7958 88) (width 0.25) (layer "F.Cu") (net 5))
 (segment (start 174.9125 88) (end 175.1425 88) (width 0.25) (layer "F.Cu") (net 5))
 (segment (start 175.7125 88) (end 178.2625 88) (width 0.25) (layer "F.Cu") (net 5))
 (segment (start 148.35 76.7) (end 148.55 76.5) (width 0.25) (layer "F.Cu") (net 6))
 (segment (start 142 79.4667) (end 142 79.7333) (width 0.25) (layer "F.Cu") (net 6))
 (segment (start 142 79.7333) (end 142 79.83) (width 0.25) (layer "F.Cu") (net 6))
 (segment (start 134.65 76.7) (end 134.88 76.7) (width 0.25) (layer "F.Cu") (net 6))
 (segment (start 134.88 76.7) (end 142 76.7) (width 0.25) (layer "F.Cu") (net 6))
 (segment (start 142 79.2) (end 142 79.4667) (width 0.25) (layer "F.Cu") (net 6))
 (segment (start 142 79.83) (end 142 80) (width 0.25) (layer "F.Cu") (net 6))
 (segment (start 142 76.7) (end 148.35 76.7) (width 0.25) (layer "F.Cu") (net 6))
 (segment (start 142 76.7) (end 142 79.2) (width 0.25) (layer "F.Cu") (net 6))
 (segment (start 106.6667 80) (end 106.3333 80) (width 0.25) (layer "F.Cu") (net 4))
 (segment (start 113.6 80) (end 107 80) (width 0.25) (layer "F.Cu") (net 4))
 (segment (start 106.3333 80) (end 106.23 80) (width 0.25) (layer "F.Cu") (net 4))
 (segment (start 107 80) (end 106.6667 80) (width 0.25) (layer "F.Cu") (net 4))
 (segment (start 106.23 80) (end 106 80) (width 0.25) (layer "F.Cu") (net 4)))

